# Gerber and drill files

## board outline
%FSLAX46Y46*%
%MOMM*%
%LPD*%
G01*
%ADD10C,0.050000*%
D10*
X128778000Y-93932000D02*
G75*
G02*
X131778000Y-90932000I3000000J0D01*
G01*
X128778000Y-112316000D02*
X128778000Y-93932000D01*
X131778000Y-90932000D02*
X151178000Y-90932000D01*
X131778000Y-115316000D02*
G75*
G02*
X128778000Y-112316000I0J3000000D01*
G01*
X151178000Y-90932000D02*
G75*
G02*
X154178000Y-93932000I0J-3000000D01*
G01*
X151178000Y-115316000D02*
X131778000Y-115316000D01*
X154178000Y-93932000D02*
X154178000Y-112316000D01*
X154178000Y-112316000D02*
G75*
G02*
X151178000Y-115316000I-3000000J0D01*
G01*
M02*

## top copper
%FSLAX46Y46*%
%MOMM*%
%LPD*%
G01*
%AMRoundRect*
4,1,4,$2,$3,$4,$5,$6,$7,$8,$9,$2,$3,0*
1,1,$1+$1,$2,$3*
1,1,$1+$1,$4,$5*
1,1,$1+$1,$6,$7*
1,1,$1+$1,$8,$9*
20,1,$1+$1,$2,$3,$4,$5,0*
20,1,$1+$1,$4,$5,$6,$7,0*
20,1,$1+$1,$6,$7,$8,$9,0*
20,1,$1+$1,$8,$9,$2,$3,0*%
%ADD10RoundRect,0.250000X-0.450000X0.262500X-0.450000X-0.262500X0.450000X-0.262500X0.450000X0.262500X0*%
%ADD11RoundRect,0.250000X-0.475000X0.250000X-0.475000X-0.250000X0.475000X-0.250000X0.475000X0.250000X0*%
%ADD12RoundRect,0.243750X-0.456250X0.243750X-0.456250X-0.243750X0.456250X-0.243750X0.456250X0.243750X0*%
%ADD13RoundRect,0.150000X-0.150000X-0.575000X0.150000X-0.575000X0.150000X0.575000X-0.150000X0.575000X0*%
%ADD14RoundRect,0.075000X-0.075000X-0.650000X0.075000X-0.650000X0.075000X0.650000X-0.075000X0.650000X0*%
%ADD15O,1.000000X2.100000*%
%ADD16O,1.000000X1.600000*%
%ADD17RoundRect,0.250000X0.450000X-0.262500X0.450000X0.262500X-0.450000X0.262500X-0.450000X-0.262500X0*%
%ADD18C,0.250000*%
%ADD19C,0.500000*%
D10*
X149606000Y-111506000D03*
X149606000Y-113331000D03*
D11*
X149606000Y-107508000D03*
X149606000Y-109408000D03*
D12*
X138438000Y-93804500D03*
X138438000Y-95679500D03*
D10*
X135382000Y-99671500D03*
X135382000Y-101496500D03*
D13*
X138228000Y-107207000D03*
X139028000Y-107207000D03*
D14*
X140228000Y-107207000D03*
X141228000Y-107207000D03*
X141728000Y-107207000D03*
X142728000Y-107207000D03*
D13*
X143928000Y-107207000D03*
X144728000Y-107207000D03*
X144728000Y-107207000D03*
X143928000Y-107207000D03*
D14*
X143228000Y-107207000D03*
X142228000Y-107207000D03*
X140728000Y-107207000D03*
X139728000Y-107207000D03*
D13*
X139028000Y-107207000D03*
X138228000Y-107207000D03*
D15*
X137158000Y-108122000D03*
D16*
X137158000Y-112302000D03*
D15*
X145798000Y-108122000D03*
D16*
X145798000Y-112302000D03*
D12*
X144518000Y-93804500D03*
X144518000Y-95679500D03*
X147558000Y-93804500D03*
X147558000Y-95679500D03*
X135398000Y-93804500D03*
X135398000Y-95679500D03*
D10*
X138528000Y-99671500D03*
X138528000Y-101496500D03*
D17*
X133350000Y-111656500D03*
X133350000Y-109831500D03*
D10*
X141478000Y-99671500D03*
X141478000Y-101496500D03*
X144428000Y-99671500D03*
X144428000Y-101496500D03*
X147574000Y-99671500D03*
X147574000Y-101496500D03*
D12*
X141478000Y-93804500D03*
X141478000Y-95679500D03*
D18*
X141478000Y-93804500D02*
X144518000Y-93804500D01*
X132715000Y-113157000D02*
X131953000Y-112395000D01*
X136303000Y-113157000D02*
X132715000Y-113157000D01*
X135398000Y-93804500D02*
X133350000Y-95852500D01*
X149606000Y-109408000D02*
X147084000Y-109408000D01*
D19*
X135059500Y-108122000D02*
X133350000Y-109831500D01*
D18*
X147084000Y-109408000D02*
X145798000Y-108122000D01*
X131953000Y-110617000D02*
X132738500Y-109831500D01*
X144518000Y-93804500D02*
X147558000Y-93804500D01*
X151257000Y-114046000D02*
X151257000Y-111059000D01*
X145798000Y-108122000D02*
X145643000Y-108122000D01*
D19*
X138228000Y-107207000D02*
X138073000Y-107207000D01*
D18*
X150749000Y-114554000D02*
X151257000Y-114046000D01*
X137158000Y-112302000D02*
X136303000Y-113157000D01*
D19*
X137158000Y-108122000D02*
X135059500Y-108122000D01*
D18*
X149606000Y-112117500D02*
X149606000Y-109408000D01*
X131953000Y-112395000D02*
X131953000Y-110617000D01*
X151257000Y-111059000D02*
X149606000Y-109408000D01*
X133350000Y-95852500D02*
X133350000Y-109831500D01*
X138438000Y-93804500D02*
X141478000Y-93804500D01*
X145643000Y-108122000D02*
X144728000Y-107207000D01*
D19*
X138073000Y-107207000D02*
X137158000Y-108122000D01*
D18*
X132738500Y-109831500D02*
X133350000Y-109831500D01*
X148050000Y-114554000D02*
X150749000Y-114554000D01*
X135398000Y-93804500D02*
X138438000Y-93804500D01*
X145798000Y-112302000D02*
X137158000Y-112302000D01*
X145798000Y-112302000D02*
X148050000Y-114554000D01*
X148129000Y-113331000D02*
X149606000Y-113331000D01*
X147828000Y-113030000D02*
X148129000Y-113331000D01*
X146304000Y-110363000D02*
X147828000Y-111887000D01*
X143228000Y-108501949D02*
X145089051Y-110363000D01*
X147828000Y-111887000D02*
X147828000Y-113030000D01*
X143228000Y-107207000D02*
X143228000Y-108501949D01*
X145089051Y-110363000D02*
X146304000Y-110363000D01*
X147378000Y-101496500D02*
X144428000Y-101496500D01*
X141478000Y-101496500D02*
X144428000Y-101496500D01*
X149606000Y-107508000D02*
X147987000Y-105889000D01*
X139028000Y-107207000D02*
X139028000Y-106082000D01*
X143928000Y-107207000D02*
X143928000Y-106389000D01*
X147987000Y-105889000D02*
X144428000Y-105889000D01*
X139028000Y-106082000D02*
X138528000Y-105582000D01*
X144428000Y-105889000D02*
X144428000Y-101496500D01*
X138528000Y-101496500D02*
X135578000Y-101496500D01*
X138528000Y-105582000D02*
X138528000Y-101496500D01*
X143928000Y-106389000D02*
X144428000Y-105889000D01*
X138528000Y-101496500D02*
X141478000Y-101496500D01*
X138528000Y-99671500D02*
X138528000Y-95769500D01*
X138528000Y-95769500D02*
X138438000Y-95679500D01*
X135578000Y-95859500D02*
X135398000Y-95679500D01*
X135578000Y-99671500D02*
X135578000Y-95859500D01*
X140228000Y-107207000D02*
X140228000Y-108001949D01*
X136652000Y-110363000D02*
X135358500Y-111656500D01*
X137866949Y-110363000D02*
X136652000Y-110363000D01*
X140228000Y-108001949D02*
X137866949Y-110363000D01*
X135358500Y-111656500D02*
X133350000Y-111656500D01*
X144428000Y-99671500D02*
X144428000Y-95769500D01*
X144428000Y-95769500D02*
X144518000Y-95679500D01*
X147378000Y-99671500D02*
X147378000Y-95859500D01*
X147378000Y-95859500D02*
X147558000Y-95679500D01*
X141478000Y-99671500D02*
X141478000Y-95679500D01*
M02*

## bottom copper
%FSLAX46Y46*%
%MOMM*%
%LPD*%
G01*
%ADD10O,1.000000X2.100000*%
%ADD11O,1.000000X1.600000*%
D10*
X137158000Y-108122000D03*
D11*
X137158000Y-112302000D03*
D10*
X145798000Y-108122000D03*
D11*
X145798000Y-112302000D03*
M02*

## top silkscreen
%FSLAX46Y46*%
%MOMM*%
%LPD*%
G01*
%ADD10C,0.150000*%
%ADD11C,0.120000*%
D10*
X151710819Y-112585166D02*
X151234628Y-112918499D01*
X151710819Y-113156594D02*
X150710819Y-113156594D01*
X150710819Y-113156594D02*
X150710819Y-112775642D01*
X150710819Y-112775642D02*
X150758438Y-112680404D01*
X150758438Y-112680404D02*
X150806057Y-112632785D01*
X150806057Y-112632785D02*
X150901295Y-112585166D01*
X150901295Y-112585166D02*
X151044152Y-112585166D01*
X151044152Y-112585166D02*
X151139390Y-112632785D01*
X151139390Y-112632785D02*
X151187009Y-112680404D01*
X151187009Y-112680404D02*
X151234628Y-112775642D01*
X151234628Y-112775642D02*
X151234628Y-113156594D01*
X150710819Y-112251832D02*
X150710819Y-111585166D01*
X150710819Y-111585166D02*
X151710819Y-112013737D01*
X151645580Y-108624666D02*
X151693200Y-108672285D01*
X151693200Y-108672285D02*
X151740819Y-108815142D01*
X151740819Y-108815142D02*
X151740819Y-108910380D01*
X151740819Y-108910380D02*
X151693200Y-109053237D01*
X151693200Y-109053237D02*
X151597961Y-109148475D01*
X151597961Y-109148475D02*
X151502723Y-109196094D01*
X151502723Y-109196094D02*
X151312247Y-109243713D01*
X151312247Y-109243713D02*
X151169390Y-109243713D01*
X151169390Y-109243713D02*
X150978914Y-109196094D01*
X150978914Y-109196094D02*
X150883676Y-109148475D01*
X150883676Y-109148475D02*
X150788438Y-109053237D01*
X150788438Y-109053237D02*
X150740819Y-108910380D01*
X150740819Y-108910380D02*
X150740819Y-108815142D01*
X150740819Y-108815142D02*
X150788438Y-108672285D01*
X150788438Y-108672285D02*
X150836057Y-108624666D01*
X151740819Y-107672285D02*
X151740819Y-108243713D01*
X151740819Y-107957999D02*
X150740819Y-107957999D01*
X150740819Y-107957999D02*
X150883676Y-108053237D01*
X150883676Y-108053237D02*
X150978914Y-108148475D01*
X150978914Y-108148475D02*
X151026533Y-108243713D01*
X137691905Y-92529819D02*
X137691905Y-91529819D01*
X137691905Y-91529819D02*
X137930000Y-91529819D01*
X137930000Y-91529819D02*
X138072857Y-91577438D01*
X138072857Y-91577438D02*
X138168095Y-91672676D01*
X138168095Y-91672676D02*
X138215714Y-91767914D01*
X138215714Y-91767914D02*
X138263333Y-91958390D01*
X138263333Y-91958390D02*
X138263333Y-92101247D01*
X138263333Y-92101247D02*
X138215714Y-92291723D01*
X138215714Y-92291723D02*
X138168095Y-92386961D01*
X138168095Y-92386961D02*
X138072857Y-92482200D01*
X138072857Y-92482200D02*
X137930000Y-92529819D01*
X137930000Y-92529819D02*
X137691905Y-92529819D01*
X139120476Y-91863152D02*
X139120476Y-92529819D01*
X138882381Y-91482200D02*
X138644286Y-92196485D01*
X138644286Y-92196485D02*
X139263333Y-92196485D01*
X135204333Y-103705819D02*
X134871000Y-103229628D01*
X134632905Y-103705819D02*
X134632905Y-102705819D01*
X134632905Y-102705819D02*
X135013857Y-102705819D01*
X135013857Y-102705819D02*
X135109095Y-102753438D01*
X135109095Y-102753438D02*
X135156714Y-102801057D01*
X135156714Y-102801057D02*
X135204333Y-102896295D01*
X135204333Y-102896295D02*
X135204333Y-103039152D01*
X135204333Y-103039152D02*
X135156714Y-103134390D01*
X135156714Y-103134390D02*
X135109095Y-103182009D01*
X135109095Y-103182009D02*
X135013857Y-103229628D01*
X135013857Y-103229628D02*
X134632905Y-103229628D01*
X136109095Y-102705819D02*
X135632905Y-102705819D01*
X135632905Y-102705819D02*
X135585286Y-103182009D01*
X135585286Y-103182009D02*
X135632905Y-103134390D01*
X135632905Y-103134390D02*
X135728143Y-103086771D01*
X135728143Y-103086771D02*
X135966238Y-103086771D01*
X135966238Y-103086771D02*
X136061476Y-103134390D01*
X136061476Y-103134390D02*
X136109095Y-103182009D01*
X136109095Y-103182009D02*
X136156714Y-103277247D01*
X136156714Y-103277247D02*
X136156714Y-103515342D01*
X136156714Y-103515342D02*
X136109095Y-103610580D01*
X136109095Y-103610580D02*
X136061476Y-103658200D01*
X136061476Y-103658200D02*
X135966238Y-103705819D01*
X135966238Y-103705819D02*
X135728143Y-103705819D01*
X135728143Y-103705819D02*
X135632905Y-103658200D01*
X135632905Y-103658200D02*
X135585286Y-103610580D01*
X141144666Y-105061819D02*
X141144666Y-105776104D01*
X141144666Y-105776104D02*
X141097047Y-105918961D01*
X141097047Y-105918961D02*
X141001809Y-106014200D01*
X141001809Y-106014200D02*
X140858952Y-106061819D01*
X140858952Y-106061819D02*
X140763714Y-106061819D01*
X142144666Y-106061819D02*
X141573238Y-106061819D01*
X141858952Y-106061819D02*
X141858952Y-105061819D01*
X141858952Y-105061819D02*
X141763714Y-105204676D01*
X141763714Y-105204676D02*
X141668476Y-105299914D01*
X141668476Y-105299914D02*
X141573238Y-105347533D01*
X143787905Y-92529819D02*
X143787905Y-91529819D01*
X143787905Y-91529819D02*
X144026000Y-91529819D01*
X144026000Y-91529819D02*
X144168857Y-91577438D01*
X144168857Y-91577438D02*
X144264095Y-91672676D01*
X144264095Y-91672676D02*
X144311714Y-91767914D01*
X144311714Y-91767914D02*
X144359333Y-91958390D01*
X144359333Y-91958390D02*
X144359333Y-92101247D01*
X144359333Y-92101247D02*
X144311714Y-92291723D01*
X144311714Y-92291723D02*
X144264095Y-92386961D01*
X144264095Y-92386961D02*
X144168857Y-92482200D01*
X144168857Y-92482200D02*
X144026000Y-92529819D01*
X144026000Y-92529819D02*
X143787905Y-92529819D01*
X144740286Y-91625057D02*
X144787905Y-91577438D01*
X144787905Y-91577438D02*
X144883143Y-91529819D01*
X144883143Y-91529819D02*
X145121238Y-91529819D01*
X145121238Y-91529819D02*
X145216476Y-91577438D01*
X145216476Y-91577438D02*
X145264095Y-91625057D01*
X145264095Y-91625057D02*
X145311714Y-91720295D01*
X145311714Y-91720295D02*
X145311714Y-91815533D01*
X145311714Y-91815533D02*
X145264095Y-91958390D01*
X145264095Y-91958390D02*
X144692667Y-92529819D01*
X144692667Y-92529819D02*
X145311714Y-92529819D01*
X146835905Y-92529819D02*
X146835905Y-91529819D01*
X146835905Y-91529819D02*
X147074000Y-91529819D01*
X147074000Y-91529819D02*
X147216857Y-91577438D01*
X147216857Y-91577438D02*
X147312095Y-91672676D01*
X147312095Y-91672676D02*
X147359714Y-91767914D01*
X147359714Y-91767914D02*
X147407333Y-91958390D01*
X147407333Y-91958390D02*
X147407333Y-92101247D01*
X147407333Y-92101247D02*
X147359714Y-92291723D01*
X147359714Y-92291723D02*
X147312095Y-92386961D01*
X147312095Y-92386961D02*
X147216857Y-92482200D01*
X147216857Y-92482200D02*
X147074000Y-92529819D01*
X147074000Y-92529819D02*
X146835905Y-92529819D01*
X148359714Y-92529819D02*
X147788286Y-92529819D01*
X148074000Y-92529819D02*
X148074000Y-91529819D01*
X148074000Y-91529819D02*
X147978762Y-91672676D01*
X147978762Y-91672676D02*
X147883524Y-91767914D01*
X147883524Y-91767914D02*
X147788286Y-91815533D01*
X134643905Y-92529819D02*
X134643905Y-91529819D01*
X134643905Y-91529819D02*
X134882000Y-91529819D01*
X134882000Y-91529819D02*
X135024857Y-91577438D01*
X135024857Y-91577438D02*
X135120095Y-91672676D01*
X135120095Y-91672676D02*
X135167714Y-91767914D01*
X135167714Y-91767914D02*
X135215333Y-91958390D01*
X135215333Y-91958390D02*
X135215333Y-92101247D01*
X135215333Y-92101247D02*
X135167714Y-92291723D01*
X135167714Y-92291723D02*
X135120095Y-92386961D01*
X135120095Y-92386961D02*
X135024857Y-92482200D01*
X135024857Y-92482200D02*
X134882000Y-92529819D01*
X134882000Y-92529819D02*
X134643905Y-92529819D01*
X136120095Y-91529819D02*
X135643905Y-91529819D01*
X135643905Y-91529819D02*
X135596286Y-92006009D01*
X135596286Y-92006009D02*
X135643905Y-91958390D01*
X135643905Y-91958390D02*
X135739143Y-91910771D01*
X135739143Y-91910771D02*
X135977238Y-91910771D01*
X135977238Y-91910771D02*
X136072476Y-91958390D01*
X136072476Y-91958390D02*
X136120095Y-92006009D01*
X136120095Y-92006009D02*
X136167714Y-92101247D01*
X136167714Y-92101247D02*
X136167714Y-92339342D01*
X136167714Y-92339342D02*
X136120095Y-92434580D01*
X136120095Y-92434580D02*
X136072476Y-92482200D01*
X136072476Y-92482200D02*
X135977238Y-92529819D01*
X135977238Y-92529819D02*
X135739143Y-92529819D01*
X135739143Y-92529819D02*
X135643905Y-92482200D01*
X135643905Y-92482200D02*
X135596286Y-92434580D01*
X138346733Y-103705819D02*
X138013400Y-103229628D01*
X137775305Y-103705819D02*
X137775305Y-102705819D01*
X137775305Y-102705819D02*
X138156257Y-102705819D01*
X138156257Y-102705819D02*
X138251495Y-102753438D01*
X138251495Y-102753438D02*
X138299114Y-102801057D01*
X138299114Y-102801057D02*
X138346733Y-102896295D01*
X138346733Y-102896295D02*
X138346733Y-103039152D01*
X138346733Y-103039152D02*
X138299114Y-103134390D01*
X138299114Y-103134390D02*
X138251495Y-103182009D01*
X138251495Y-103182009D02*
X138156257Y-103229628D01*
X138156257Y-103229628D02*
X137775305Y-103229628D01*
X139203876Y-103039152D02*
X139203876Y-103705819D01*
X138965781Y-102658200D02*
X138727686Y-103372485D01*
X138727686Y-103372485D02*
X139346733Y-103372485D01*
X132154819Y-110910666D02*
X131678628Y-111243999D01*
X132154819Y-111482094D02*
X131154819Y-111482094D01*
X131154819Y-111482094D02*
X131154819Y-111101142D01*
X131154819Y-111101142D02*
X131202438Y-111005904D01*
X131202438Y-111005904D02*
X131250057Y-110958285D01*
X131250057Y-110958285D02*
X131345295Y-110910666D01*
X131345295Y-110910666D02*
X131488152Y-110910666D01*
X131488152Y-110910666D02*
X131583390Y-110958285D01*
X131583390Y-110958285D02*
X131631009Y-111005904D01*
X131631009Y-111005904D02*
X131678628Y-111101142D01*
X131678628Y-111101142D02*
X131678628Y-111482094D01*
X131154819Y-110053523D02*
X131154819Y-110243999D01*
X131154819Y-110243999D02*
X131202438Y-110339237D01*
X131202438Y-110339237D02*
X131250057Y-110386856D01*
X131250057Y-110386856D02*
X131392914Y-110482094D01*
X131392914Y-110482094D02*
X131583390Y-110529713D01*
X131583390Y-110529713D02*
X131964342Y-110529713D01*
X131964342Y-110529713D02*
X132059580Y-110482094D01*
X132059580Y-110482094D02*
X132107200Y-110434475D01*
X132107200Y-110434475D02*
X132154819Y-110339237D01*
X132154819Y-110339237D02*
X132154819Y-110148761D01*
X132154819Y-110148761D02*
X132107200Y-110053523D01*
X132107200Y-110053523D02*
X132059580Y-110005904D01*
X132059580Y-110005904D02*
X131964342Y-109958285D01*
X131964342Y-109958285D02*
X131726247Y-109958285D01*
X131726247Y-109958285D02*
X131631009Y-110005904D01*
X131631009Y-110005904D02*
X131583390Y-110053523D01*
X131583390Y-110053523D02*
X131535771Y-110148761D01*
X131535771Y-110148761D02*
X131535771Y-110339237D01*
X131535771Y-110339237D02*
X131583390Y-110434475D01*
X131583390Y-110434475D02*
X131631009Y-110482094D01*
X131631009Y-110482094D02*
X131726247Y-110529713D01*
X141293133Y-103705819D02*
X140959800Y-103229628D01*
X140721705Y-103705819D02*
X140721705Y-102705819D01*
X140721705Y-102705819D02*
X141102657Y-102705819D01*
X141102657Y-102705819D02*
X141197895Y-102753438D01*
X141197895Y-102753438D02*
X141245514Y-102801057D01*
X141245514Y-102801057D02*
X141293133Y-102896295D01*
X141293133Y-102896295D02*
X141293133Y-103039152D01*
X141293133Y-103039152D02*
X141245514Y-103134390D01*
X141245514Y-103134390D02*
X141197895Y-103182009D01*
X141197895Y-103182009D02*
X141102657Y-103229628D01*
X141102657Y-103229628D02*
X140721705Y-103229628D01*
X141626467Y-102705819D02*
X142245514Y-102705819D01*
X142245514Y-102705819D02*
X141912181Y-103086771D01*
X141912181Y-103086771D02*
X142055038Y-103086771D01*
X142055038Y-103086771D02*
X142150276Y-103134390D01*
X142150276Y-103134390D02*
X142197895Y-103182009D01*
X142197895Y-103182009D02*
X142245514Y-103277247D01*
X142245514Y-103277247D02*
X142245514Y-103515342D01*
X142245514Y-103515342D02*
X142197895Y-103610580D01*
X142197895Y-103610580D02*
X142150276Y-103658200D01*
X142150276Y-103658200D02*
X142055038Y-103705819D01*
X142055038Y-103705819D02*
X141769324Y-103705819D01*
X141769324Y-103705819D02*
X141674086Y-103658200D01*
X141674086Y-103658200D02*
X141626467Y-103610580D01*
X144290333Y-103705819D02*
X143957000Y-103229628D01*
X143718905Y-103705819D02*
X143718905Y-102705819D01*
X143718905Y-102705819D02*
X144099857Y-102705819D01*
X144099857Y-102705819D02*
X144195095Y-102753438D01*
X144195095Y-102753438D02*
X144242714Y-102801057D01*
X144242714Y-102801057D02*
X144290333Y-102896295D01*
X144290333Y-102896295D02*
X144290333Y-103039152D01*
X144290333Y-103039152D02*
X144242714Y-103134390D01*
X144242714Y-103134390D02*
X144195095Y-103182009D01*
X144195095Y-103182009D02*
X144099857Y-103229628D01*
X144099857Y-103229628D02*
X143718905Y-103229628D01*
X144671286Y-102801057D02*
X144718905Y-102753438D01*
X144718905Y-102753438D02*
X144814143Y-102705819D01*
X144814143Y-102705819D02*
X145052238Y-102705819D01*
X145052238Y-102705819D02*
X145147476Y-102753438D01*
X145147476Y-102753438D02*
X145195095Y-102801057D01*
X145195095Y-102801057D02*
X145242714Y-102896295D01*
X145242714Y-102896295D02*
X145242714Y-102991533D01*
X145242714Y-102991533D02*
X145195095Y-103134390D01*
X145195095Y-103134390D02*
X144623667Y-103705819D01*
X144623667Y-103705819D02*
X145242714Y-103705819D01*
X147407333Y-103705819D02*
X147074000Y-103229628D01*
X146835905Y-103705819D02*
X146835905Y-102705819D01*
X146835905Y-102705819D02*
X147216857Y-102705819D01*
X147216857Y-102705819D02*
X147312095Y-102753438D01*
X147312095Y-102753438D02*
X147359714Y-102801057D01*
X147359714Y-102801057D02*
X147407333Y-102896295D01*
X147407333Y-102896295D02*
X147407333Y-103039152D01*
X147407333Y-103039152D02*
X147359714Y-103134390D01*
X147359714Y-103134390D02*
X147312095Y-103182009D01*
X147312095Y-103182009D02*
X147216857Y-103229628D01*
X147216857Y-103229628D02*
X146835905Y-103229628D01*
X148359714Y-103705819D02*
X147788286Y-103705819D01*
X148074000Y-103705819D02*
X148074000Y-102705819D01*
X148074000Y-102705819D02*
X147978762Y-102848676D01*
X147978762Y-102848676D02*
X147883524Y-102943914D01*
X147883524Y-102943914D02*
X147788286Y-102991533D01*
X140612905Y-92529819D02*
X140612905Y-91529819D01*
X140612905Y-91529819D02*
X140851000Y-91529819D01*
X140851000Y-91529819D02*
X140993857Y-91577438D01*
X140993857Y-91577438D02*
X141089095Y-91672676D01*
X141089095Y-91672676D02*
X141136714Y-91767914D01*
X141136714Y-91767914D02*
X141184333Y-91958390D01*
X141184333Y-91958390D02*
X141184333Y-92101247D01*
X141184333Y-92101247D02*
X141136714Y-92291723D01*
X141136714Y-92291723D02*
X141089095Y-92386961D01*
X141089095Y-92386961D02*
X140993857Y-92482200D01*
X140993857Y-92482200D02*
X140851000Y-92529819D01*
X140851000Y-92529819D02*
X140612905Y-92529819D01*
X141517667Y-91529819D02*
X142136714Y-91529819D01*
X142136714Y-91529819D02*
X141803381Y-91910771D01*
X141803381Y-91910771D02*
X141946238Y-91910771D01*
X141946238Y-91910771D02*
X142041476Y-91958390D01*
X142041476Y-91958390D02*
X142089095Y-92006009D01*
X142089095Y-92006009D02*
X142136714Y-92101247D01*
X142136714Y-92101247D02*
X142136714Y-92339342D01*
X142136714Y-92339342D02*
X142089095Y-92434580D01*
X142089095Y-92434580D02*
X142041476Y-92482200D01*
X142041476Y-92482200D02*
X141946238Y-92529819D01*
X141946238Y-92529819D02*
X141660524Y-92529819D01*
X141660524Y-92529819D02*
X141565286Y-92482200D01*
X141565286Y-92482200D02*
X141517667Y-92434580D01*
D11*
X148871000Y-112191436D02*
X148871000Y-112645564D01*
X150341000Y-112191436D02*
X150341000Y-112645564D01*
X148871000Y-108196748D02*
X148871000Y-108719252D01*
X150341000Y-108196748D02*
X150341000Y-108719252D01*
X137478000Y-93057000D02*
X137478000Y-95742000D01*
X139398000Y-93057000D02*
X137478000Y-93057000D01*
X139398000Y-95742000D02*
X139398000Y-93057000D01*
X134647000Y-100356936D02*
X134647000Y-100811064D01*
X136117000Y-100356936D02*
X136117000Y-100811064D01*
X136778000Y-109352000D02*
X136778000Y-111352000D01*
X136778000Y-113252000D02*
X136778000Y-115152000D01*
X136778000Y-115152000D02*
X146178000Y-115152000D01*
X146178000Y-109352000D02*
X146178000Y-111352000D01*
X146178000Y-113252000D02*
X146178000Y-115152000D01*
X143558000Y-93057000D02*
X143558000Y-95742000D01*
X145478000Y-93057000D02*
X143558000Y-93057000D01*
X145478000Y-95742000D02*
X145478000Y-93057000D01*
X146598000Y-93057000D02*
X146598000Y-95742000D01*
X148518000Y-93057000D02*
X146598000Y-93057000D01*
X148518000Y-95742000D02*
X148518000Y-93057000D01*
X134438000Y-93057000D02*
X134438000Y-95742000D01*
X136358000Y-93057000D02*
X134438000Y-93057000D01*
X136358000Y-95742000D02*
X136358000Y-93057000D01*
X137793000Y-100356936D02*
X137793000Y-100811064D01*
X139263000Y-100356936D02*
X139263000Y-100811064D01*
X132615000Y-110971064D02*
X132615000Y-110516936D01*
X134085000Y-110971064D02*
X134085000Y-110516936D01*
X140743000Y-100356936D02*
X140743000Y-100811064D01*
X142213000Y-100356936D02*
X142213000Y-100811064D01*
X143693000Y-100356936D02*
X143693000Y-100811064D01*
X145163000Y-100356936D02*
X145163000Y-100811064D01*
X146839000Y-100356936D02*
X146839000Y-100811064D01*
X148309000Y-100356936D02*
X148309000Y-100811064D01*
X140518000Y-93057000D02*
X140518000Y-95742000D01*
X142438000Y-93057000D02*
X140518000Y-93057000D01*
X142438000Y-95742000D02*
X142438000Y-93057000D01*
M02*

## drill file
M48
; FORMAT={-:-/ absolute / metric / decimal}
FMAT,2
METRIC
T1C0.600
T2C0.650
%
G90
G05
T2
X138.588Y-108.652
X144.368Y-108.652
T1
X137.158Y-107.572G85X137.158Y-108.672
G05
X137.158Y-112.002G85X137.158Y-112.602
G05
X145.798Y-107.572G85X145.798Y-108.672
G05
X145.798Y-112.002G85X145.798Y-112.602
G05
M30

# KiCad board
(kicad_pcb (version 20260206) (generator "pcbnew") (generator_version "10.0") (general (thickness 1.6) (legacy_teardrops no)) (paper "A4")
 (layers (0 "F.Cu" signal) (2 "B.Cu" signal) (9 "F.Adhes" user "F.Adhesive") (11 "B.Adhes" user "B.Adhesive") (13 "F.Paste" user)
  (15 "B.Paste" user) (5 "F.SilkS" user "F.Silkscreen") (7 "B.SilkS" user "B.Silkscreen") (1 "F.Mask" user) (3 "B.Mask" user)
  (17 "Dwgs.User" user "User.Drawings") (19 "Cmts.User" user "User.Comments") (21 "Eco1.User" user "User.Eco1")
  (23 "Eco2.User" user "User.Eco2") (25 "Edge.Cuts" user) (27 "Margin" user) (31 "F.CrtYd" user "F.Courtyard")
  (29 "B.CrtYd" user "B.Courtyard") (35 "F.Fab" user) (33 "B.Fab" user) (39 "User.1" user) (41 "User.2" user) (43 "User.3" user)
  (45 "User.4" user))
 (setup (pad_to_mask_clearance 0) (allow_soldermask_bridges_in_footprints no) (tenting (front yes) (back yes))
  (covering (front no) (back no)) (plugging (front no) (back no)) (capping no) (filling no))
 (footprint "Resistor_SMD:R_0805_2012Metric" (layer "F.Cu") (at 149.606 112.4185 -90)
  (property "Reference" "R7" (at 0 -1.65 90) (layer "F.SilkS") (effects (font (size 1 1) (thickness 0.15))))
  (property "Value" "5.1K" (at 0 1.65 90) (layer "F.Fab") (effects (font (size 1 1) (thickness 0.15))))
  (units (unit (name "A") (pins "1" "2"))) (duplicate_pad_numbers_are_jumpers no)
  (fp_line (start -0.227064 0.735) (end 0.227064 0.735) (stroke (width 0.12) (type solid)) (layer "F.SilkS"))
  (fp_line (start -0.227064 -0.735) (end 0.227064 -0.735) (stroke (width 0.12) (type solid)) (layer "F.SilkS"))
  (pad "1" smd roundrect (at -0.9125 0 270) (size 1.025 1.4) (layers "F.Cu" "F.Mask" "F.Paste") (roundrect_rratio 0.243902) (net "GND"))
  (pad "2" smd roundrect (at 0.9125 0 270) (size 1.025 1.4) (layers "F.Cu" "F.Mask" "F.Paste") (roundrect_rratio 0.243902)
   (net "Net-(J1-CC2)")))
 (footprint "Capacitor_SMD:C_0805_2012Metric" (layer "F.Cu") (at 149.606 108.458 -90)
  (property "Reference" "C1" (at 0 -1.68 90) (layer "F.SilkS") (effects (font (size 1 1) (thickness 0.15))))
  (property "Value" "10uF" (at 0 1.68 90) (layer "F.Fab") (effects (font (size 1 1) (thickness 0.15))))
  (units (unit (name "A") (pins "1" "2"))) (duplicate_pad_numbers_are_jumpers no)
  (fp_line (start -0.261252 0.735) (end 0.261252 0.735) (stroke (width 0.12) (type solid)) (layer "F.SilkS"))
  (fp_line (start -0.261252 -0.735) (end 0.261252 -0.735) (stroke (width 0.12) (type solid)) (layer "F.SilkS"))
  (pad "1" smd roundrect (at -0.95 0 270) (size 1 1.45) (layers "F.Cu" "F.Mask" "F.Paste") (roundrect_rratio 0.25) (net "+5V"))
  (pad "2" smd roundrect (at 0.95 0 270) (size 1 1.45) (layers "F.Cu" "F.Mask" "F.Paste") (roundrect_rratio 0.25) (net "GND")))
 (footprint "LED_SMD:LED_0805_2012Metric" (layer "F.Cu") (at 138.438 94.742 -90)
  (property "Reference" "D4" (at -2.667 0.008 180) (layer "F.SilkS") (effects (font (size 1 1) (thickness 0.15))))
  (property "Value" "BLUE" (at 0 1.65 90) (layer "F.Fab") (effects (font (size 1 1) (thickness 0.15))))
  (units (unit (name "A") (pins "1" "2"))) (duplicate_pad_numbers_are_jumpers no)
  (fp_line (start -1.685 0.96) (end 1 0.96) (stroke (width 0.12) (type solid)) (layer "F.SilkS"))
  (fp_line (start -1.685 -0.96) (end -1.685 0.96) (stroke (width 0.12) (type solid)) (layer "F.SilkS"))
  (fp_line (start 1 -0.96) (end -1.685 -0.96) (stroke (width 0.12) (type solid)) (layer "F.SilkS"))
  (pad "1" smd roundrect (at -0.9375 0 270) (size 0.975 1.4) (layers "F.Cu" "F.Mask" "F.Paste") (roundrect_rratio 0.25) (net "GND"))
  (pad "2" smd roundrect (at 0.9375 0 270) (size 0.975 1.4) (layers "F.Cu" "F.Mask" "F.Paste") (roundrect_rratio 0.25) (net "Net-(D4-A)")))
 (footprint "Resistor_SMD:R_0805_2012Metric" (layer "F.Cu") (at 135.382 100.584 -90)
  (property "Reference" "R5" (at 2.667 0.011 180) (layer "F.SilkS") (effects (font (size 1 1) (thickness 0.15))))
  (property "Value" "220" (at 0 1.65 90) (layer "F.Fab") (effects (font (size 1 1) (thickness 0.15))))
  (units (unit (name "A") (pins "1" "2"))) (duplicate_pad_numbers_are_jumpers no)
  (fp_line (start -0.227064 0.735) (end 0.227064 0.735) (stroke (width 0.12) (type solid)) (layer "F.SilkS"))
  (fp_line (start -0.227064 -0.735) (end 0.227064 -0.735) (stroke (width 0.12) (type solid)) (layer "F.SilkS"))
  (pad "1" smd roundrect (at -0.9125 0 270) (size 1.025 1.4) (layers "F.Cu" "F.Mask" "F.Paste") (roundrect_rratio 0.243902)
   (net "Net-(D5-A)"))
  (pad "2" smd roundrect (at 0.9125 0 270) (size 1.025 1.4) (layers "F.Cu" "F.Mask" "F.Paste") (roundrect_rratio 0.243902) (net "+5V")))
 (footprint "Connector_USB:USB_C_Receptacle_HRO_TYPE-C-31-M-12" (layer "F.Cu") (at 141.478 111.252)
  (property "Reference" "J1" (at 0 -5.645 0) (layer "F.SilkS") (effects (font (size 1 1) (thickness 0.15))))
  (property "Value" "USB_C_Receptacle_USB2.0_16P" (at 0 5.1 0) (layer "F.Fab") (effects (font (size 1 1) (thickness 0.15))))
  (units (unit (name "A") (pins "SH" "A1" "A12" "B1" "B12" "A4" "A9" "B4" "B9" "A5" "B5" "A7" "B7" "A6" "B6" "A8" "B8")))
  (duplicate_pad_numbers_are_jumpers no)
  (fp_line (start -4.7 -1.9) (end -4.7 0.1) (stroke (width 0.12) (type solid)) (layer "F.SilkS"))
  (fp_line (start -4.7 2) (end -4.7 3.9) (stroke (width 0.12) (type solid)) (layer "F.SilkS"))
  (fp_line (start -4.7 3.9) (end 4.7 3.9) (stroke (width 0.12) (type solid)) (layer "F.SilkS"))
  (fp_line (start 4.7 -1.9) (end 4.7 0.1) (stroke (width 0.12) (type solid)) (layer "F.SilkS"))
  (fp_line (start 4.7 2) (end 4.7 3.9) (stroke (width 0.12) (type solid)) (layer "F.SilkS"))
  (pad "" np_thru_hole circle (at -2.89 -2.6) (size 0.65 0.65) (drill 0.65) (layers "*.Cu" "*.Mask"))
  (pad "" np_thru_hole circle (at 2.89 -2.6) (size 0.65 0.65) (drill 0.65) (layers "*.Cu" "*.Mask"))
  (pad "A1" smd roundrect (at -3.25 -4.045) (size 0.6 1.45) (layers "F.Cu" "F.Mask" "F.Paste") (roundrect_rratio 0.25) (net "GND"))
  (pad "A4" smd roundrect (at -2.45 -4.045) (size 0.6 1.45) (layers "F.Cu" "F.Mask" "F.Paste") (roundrect_rratio 0.25) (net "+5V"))
  (pad "A5" smd roundrect (at -1.25 -4.045) (size 0.3 1.45) (layers "F.Cu" "F.Mask" "F.Paste") (roundrect_rratio 0.25) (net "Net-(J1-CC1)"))
  (pad "A6" smd roundrect (at -0.25 -4.045) (size 0.3 1.45) (layers "F.Cu" "F.Mask" "F.Paste") (roundrect_rratio 0.25)
   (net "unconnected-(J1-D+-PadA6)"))
  (pad "A7" smd roundrect (at 0.25 -4.045) (size 0.3 1.45) (layers "F.Cu" "F.Mask" "F.Paste") (roundrect_rratio 0.25)
   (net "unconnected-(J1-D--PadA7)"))
  (pad "A8" smd roundrect (at 1.25 -4.045) (size 0.3 1.45) (layers "F.Cu" "F.Mask" "F.Paste") (roundrect_rratio 0.25)
   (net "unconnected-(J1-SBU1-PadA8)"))
  (pad "A9" smd roundrect (at 2.45 -4.045) (size 0.6 1.45) (layers "F.Cu" "F.Mask" "F.Paste") (roundrect_rratio 0.25) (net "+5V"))
  (pad "A12" smd roundrect (at 3.25 -4.045) (size 0.6 1.45) (layers "F.Cu" "F.Mask" "F.Paste") (roundrect_rratio 0.25) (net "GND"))
  (pad "B1" smd roundrect (at 3.25 -4.045) (size 0.6 1.45) (layers "F.Cu" "F.Mask" "F.Paste") (roundrect_rratio 0.25) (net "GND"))
  (pad "B4" smd roundrect (at 2.45 -4.045) (size 0.6 1.45) (layers "F.Cu" "F.Mask" "F.Paste") (roundrect_rratio 0.25) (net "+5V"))
  (pad "B5" smd roundrect (at 1.75 -4.045) (size 0.3 1.45) (layers "F.Cu" "F.Mask" "F.Paste") (roundrect_rratio 0.25) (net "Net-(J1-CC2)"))
  (pad "B6" smd roundrect (at 0.75 -4.045) (size 0.3 1.45) (layers "F.Cu" "F.Mask" "F.Paste") (roundrect_rratio 0.25)
   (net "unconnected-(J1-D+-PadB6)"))
  (pad "B7" smd roundrect (at -0.75 -4.045) (size 0.3 1.45) (layers "F.Cu" "F.Mask" "F.Paste") (roundrect_rratio 0.25)
   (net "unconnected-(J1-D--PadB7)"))
  (pad "B8" smd roundrect (at -1.75 -4.045) (size 0.3 1.45) (layers "F.Cu" "F.Mask" "F.Paste") (roundrect_rratio 0.25)
   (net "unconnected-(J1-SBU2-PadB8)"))
  (pad "B9" smd roundrect (at -2.45 -4.045) (size 0.6 1.45) (layers "F.Cu" "F.Mask" "F.Paste") (roundrect_rratio 0.25) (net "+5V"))
  (pad "B12" smd roundrect (at -3.25 -4.045) (size 0.6 1.45) (layers "F.Cu" "F.Mask" "F.Paste") (roundrect_rratio 0.25) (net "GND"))
  (pad "SH" thru_hole oval (at -4.32 -3.13) (size 1 2.1) (drill oval 0.6 1.7) (layers "*.Cu" "*.Mask") (remove_unused_layers no) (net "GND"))
  (pad "SH" thru_hole oval (at -4.32 1.05) (size 1 1.6) (drill oval 0.6 1.2) (layers "*.Cu" "*.Mask") (remove_unused_layers no) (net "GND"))
  (pad "SH" thru_hole oval (at 4.32 -3.13) (size 1 2.1) (drill oval 0.6 1.7) (layers "*.Cu" "*.Mask") (remove_unused_layers no) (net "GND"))
  (pad "SH" thru_hole oval (at 4.32 1.05) (size 1 1.6) (drill oval 0.6 1.2) (layers "*.Cu" "*.Mask") (remove_unused_layers no) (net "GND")))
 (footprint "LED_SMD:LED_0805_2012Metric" (layer "F.Cu") (at 144.518 94.742 -90)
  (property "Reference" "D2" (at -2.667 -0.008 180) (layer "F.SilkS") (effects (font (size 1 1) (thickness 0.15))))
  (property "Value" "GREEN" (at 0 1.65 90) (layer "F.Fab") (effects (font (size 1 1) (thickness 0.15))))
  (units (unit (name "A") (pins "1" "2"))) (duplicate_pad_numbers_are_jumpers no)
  (fp_line (start -1.685 0.96) (end 1 0.96) (stroke (width 0.12) (type solid)) (layer "F.SilkS"))
  (fp_line (start -1.685 -0.96) (end -1.685 0.96) (stroke (width 0.12) (type solid)) (layer "F.SilkS"))
  (fp_line (start 1 -0.96) (end -1.685 -0.96) (stroke (width 0.12) (type solid)) (layer "F.SilkS"))
  (pad "1" smd roundrect (at -0.9375 0 270) (size 0.975 1.4) (layers "F.Cu" "F.Mask" "F.Paste") (roundrect_rratio 0.25) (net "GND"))
  (pad "2" smd roundrect (at 0.9375 0 270) (size 0.975 1.4) (layers "F.Cu" "F.Mask" "F.Paste") (roundrect_rratio 0.25) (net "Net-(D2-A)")))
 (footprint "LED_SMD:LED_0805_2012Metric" (layer "F.Cu") (at 147.558 94.742 -90)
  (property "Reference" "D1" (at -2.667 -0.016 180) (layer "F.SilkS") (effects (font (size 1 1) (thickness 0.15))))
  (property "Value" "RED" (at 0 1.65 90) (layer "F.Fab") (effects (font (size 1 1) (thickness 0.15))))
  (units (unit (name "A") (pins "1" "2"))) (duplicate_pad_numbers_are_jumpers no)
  (fp_line (start -1.685 0.96) (end 1 0.96) (stroke (width 0.12) (type solid)) (layer "F.SilkS"))
  (fp_line (start -1.685 -0.96) (end -1.685 0.96) (stroke (width 0.12) (type solid)) (layer "F.SilkS"))
  (fp_line (start 1 -0.96) (end -1.685 -0.96) (stroke (width 0.12) (type solid)) (layer "F.SilkS"))
  (pad "1" smd roundrect (at -0.9375 0 270) (size 0.975 1.4) (layers "F.Cu" "F.Mask" "F.Paste") (roundrect_rratio 0.25) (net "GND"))
  (pad "2" smd roundrect (at 0.9375 0 270) (size 0.975 1.4) (layers "F.Cu" "F.Mask" "F.Paste") (roundrect_rratio 0.25) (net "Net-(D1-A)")))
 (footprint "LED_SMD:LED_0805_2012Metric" (layer "F.Cu") (at 135.398 94.742 -90)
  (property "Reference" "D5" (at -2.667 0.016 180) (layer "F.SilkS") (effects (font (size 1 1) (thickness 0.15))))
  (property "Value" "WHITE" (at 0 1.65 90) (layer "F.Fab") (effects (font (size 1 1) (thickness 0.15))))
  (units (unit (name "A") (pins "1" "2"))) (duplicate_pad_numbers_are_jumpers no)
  (fp_line (start -1.685 0.96) (end 1 0.96) (stroke (width 0.12) (type solid)) (layer "F.SilkS"))
  (fp_line (start -1.685 -0.96) (end -1.685 0.96) (stroke (width 0.12) (type solid)) (layer "F.SilkS"))
  (fp_line (start 1 -0.96) (end -1.685 -0.96) (stroke (width 0.12) (type solid)) (layer "F.SilkS"))
  (pad "1" smd roundrect (at -0.9375 0 270) (size 0.975 1.4) (layers "F.Cu" "F.Mask" "F.Paste") (roundrect_rratio 0.25) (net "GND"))
  (pad "2" smd roundrect (at 0.9375 0 270) (size 0.975 1.4) (layers "F.Cu" "F.Mask" "F.Paste") (roundrect_rratio 0.25) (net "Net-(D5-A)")))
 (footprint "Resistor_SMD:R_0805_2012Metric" (layer "F.Cu") (at 138.528 100.584 -90)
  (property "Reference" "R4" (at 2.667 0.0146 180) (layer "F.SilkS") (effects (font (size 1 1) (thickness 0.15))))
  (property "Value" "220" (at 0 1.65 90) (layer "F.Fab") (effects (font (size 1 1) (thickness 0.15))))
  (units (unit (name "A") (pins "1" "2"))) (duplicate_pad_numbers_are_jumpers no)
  (fp_line (start -0.227064 0.735) (end 0.227064 0.735) (stroke (width 0.12) (type solid)) (layer "F.SilkS"))
  (fp_line (start -0.227064 -0.735) (end 0.227064 -0.735) (stroke (width 0.12) (type solid)) (layer "F.SilkS"))
  (pad "1" smd roundrect (at -0.9125 0 270) (size 1.025 1.4) (layers "F.Cu" "F.Mask" "F.Paste") (roundrect_rratio 0.243902)
   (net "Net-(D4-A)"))
  (pad "2" smd roundrect (at 0.9125 0 270) (size 1.025 1.4) (layers "F.Cu" "F.Mask" "F.Paste") (roundrect_rratio 0.243902) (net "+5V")))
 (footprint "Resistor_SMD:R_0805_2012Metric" (layer "F.Cu") (at 133.35 110.744 90)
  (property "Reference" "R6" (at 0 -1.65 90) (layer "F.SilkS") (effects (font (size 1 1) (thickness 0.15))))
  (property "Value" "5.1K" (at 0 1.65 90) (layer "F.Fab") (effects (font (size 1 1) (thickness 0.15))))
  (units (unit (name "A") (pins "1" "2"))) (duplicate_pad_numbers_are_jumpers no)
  (fp_line (start -0.227064 -0.735) (end 0.227064 -0.735) (stroke (width 0.12) (type solid)) (layer "F.SilkS"))
  (fp_line (start -0.227064 0.735) (end 0.227064 0.735) (stroke (width 0.12) (type solid)) (layer "F.SilkS"))
  (pad "1" smd roundrect (at -0.9125 0 90) (size 1.025 1.4) (layers "F.Cu" "F.Mask" "F.Paste") (roundrect_rratio 0.243902)
   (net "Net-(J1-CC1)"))
  (pad "2" smd roundrect (at 0.9125 0 90) (size 1.025 1.4) (layers "F.Cu" "F.Mask" "F.Paste") (roundrect_rratio 0.243902) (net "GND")))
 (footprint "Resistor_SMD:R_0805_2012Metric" (layer "F.Cu") (at 141.478 100.584 -90)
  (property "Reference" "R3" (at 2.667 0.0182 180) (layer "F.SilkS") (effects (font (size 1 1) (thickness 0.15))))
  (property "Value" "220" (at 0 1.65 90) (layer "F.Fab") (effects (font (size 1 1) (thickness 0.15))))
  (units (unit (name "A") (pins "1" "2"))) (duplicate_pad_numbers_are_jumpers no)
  (fp_line (start -0.227064 0.735) (end 0.227064 0.735) (stroke (width 0.12) (type solid)) (layer "F.SilkS"))
  (fp_line (start -0.227064 -0.735) (end 0.227064 -0.735) (stroke (width 0.12) (type solid)) (layer "F.SilkS"))
  (pad "1" smd roundrect (at -0.9125 0 270) (size 1.025 1.4) (layers "F.Cu" "F.Mask" "F.Paste") (roundrect_rratio 0.243902)
   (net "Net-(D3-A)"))
  (pad "2" smd roundrect (at 0.9125 0 270) (size 1.025 1.4) (layers "F.Cu" "F.Mask" "F.Paste") (roundrect_rratio 0.243902) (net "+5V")))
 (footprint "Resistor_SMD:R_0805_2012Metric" (layer "F.Cu") (at 144.428 100.584 -90)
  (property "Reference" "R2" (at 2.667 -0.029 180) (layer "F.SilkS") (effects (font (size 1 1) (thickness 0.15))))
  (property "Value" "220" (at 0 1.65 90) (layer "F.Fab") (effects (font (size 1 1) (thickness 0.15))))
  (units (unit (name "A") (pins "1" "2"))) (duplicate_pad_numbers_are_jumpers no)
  (fp_line (start -0.227064 0.735) (end 0.227064 0.735) (stroke (width 0.12) (type solid)) (layer "F.SilkS"))
  (fp_line (start -0.227064 -0.735) (end 0.227064 -0.735) (stroke (width 0.12) (type solid)) (layer "F.SilkS"))
  (pad "1" smd roundrect (at -0.9125 0 270) (size 1.025 1.4) (layers "F.Cu" "F.Mask" "F.Paste") (roundrect_rratio 0.243902)
   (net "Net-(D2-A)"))
  (pad "2" smd roundrect (at 0.9125 0 270) (size 1.025 1.4) (layers "F.Cu" "F.Mask" "F.Paste") (roundrect_rratio 0.243902) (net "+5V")))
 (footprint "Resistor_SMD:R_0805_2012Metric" (layer "F.Cu") (at 147.574 100.584 -90)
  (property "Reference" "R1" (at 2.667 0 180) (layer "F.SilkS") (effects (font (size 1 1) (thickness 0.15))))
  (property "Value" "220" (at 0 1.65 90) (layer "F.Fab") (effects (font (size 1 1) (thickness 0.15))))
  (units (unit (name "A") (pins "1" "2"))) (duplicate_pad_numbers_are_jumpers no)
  (fp_line (start -0.227064 0.735) (end 0.227064 0.735) (stroke (width 0.12) (type solid)) (layer "F.SilkS"))
  (fp_line (start -0.227064 -0.735) (end 0.227064 -0.735) (stroke (width 0.12) (type solid)) (layer "F.SilkS"))
  (pad "1" smd roundrect (at -0.9125 0 270) (size 1.025 1.4) (layers "F.Cu" "F.Mask" "F.Paste") (roundrect_rratio 0.243902)
   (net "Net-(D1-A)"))
  (pad "2" smd roundrect (at 0.9125 0 270) (size 1.025 1.4) (layers "F.Cu" "F.Mask" "F.Paste") (roundrect_rratio 0.243902) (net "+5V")))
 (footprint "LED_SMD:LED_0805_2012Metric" (layer "F.Cu") (at 141.478 94.742 -90)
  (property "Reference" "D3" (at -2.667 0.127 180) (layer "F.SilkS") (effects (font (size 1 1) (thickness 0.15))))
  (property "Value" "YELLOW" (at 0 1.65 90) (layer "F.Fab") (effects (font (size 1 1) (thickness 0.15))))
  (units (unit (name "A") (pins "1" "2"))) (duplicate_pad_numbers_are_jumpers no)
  (fp_line (start -1.685 0.96) (end 1 0.96) (stroke (width 0.12) (type solid)) (layer "F.SilkS"))
  (fp_line (start -1.685 -0.96) (end -1.685 0.96) (stroke (width 0.12) (type solid)) (layer "F.SilkS"))
  (fp_line (start 1 -0.96) (end -1.685 -0.96) (stroke (width 0.12) (type solid)) (layer "F.SilkS"))
  (pad "1" smd roundrect (at -0.9375 0 270) (size 0.975 1.4) (layers "F.Cu" "F.Mask" "F.Paste") (roundrect_rratio 0.25) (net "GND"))
  (pad "2" smd roundrect (at 0.9375 0 270) (size 0.975 1.4) (layers "F.Cu" "F.Mask" "F.Paste") (roundrect_rratio 0.25) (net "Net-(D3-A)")))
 (gr_arc (start 128.778 93.932) (mid 129.65668 91.81068) (end 131.778 90.932) (stroke (width 0.05) (type default)) (layer "Edge.Cuts"))
 (gr_line (start 128.778 112.316) (end 128.778 93.932) (stroke (width 0.05) (type default)) (layer "Edge.Cuts"))
 (gr_line (start 131.778 90.932) (end 151.178 90.932) (stroke (width 0.05) (type default)) (layer "Edge.Cuts"))
 (gr_arc (start 131.778 115.316) (mid 129.65668 114.43732) (end 128.778 112.316) (stroke (width 0.05) (type default)) (layer "Edge.Cuts"))
 (gr_arc (start 151.178 90.932) (mid 153.29932 91.81068) (end 154.178 93.932) (stroke (width 0.05) (type default)) (layer "Edge.Cuts"))
 (gr_line (start 151.178 115.316) (end 131.778 115.316) (stroke (width 0.05) (type default)) (layer "Edge.Cuts"))
 (gr_line (start 154.178 93.932) (end 154.178 112.316) (stroke (width 0.05) (type default)) (layer "Edge.Cuts"))
 (gr_arc (start 154.178 112.316) (mid 153.29932 114.43732) (end 151.178 115.316) (stroke (width 0.05) (type default)) (layer "Edge.Cuts"))
 (segment (start 141.478 93.8045) (end 144.518 93.8045) (width 0.25) (layer "F.Cu") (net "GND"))
 (segment (start 132.715 113.157) (end 131.953 112.395) (width 0.25) (layer "F.Cu") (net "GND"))
 (segment (start 136.303 113.157) (end 132.715 113.157) (width 0.25) (layer "F.Cu") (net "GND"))
 (segment (start 135.398 93.8045) (end 133.35 95.8525) (width 0.25) (layer "F.Cu") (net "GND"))
 (segment (start 149.606 109.408) (end 147.084 109.408) (width 0.25) (layer "F.Cu") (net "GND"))
 (segment (start 135.0595 108.122) (end 133.35 109.8315) (width 0.5) (layer "F.Cu") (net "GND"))
 (segment (start 147.084 109.408) (end 145.798 108.122) (width 0.25) (layer "F.Cu") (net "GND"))
 (segment (start 131.953 110.617) (end 132.7385 109.8315) (width 0.25) (layer "F.Cu") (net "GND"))
 (segment (start 144.518 93.8045) (end 147.558 93.8045) (width 0.25) (layer "F.Cu") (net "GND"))
 (segment (start 151.257 114.046) (end 151.257 111.059) (width 0.25) (layer "F.Cu") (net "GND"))
 (segment (start 145.798 108.122) (end 145.643 108.122) (width 0.25) (layer "F.Cu") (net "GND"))
 (segment (start 138.228 107.207) (end 138.073 107.207) (width 0.5) (layer "F.Cu") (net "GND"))
 (segment (start 150.749 114.554) (end 151.257 114.046) (width 0.25) (layer "F.Cu") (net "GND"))
 (segment (start 137.158 112.302) (end 136.303 113.157) (width 0.25) (layer "F.Cu") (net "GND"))
 (segment (start 137.158 108.122) (end 135.0595 108.122) (width 0.5) (layer "F.Cu") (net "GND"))
 (segment (start 149.606 112.1175) (end 149.606 109.408) (width 0.25) (layer "F.Cu") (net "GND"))
 (segment (start 131.953 112.395) (end 131.953 110.617) (width 0.25) (layer "F.Cu") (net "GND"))
 (segment (start 151.257 111.059) (end 149.606 109.408) (width 0.25) (layer "F.Cu") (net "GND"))
 (segment (start 133.35 95.8525) (end 133.35 109.8315) (width 0.25) (layer "F.Cu") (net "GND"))
 (segment (start 138.438 93.8045) (end 141.478 93.8045) (width 0.25) (layer "F.Cu") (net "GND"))
 (segment (start 145.643 108.122) (end 144.728 107.207) (width 0.25) (layer "F.Cu") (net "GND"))
 (segment (start 138.073 107.207) (end 137.158 108.122) (width 0.5) (layer "F.Cu") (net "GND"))
 (segment (start 132.7385 109.8315) (end 133.35 109.8315) (width 0.25) (layer "F.Cu") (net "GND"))
 (segment (start 148.05 114.554) (end 150.749 114.554) (width 0.25) (layer "F.Cu") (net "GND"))
 (segment (start 135.398 93.8045) (end 138.438 93.8045) (width 0.25) (layer "F.Cu") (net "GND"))
 (segment (start 145.798 112.302) (end 137.158 112.302) (width 0.25) (layer "F.Cu") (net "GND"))
 (segment (start 145.798 112.302) (end 148.05 114.554) (width 0.25) (layer "F.Cu") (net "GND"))
 (segment (start 148.129 113.331) (end 149.606 113.331) (width 0.25) (layer "F.Cu") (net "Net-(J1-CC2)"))
 (segment (start 147.828 113.03) (end 148.129 113.331) (width 0.25) (layer "F.Cu") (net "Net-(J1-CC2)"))
 (segment (start 146.304 110.363) (end 147.828 111.887) (width 0.25) (layer "F.Cu") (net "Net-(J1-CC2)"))
 (segment (start 143.228 108.501949) (end 145.089051 110.363) (width 0.25) (layer "F.Cu") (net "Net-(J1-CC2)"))
 (segment (start 147.828 111.887) (end 147.828 113.03) (width 0.25) (layer "F.Cu") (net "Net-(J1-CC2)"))
 (segment (start 143.228 107.207) (end 143.228 108.501949) (width 0.25) (layer "F.Cu") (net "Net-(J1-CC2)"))
 (segment (start 145.089051 110.363) (end 146.304 110.363) (width 0.25) (layer "F.Cu") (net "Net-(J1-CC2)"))
 (segment (start 147.378 101.4965) (end 144.428 101.4965) (width 0.25) (layer "F.Cu") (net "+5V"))
 (segment (start 141.478 101.4965) (end 144.428 101.4965) (width 0.25) (layer "F.Cu") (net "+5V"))
 (segment (start 149.606 107.508) (end 147.987 105.889) (width 0.25) (layer "F.Cu") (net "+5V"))
 (segment (start 139.028 107.207) (end 139.028 106.082) (width 0.25) (layer "F.Cu") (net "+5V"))
 (segment (start 143.928 107.207) (end 143.928 106.389) (width 0.25) (layer "F.Cu") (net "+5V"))
 (segment (start 147.987 105.889) (end 144.428 105.889) (width 0.25) (layer "F.Cu") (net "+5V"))
 (segment (start 139.028 106.082) (end 138.528 105.582) (width 0.25) (layer "F.Cu") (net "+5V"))
 (segment (start 144.428 105.889) (end 144.428 101.4965) (width 0.25) (layer "F.Cu") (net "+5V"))
 (segment (start 138.528 101.4965) (end 135.578 101.4965) (width 0.25) (layer "F.Cu") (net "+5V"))
 (segment (start 138.528 105.582) (end 138.528 101.4965) (width 0.25) (layer "F.Cu") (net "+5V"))
 (segment (start 143.928 106.389) (end 144.428 105.889) (width 0.25) (layer "F.Cu") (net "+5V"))
 (segment (start 138.528 101.4965) (end 141.478 101.4965) (width 0.25) (layer "F.Cu") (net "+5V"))
 (segment (start 138.528 99.6715) (end 138.528 95.7695) (width 0.25) (layer "F.Cu") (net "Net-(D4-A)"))
 (segment (start 138.528 95.7695) (end 138.438 95.6795) (width 0.25) (layer "F.Cu") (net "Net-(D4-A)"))
 (segment (start 135.578 95.8595) (end 135.398 95.6795) (width 0.25) (layer "F.Cu") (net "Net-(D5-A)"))
 (segment (start 135.578 99.6715) (end 135.578 95.8595) (width 0.25) (layer "F.Cu") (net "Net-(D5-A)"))
 (segment (start 140.228 107.207) (end 140.228 108.001949) (width 0.25) (layer "F.Cu") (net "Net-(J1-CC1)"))
 (segment (start 136.652 110.363) (end 135.3585 111.6565) (width 0.25) (layer "F.Cu") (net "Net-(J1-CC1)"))
 (segment (start 137.866949 110.363) (end 136.652 110.363) (width 0.25) (layer "F.Cu") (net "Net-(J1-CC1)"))
 (segment (start 140.228 108.001949) (end 137.866949 110.363) (width 0.25) (layer "F.Cu") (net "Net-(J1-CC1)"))
 (segment (start 135.3585 111.6565) (end 133.35 111.6565) (width 0.25) (layer "F.Cu") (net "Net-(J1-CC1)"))
 (segment (start 144.428 99.6715) (end 144.428 95.7695) (width 0.25) (layer "F.Cu") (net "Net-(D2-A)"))
 (segment (start 144.428 95.7695) (end 144.518 95.6795) (width 0.25) (layer "F.Cu") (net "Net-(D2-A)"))
 (segment (start 147.378 99.6715) (end 147.378 95.8595) (width 0.25) (layer "F.Cu") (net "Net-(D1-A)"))
 (segment (start 147.378 95.8595) (end 147.558 95.6795) (width 0.25) (layer "F.Cu") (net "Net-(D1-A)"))
 (segment (start 141.478 99.6715) (end 141.478 95.6795) (width 0.25) (layer "F.Cu") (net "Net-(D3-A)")))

